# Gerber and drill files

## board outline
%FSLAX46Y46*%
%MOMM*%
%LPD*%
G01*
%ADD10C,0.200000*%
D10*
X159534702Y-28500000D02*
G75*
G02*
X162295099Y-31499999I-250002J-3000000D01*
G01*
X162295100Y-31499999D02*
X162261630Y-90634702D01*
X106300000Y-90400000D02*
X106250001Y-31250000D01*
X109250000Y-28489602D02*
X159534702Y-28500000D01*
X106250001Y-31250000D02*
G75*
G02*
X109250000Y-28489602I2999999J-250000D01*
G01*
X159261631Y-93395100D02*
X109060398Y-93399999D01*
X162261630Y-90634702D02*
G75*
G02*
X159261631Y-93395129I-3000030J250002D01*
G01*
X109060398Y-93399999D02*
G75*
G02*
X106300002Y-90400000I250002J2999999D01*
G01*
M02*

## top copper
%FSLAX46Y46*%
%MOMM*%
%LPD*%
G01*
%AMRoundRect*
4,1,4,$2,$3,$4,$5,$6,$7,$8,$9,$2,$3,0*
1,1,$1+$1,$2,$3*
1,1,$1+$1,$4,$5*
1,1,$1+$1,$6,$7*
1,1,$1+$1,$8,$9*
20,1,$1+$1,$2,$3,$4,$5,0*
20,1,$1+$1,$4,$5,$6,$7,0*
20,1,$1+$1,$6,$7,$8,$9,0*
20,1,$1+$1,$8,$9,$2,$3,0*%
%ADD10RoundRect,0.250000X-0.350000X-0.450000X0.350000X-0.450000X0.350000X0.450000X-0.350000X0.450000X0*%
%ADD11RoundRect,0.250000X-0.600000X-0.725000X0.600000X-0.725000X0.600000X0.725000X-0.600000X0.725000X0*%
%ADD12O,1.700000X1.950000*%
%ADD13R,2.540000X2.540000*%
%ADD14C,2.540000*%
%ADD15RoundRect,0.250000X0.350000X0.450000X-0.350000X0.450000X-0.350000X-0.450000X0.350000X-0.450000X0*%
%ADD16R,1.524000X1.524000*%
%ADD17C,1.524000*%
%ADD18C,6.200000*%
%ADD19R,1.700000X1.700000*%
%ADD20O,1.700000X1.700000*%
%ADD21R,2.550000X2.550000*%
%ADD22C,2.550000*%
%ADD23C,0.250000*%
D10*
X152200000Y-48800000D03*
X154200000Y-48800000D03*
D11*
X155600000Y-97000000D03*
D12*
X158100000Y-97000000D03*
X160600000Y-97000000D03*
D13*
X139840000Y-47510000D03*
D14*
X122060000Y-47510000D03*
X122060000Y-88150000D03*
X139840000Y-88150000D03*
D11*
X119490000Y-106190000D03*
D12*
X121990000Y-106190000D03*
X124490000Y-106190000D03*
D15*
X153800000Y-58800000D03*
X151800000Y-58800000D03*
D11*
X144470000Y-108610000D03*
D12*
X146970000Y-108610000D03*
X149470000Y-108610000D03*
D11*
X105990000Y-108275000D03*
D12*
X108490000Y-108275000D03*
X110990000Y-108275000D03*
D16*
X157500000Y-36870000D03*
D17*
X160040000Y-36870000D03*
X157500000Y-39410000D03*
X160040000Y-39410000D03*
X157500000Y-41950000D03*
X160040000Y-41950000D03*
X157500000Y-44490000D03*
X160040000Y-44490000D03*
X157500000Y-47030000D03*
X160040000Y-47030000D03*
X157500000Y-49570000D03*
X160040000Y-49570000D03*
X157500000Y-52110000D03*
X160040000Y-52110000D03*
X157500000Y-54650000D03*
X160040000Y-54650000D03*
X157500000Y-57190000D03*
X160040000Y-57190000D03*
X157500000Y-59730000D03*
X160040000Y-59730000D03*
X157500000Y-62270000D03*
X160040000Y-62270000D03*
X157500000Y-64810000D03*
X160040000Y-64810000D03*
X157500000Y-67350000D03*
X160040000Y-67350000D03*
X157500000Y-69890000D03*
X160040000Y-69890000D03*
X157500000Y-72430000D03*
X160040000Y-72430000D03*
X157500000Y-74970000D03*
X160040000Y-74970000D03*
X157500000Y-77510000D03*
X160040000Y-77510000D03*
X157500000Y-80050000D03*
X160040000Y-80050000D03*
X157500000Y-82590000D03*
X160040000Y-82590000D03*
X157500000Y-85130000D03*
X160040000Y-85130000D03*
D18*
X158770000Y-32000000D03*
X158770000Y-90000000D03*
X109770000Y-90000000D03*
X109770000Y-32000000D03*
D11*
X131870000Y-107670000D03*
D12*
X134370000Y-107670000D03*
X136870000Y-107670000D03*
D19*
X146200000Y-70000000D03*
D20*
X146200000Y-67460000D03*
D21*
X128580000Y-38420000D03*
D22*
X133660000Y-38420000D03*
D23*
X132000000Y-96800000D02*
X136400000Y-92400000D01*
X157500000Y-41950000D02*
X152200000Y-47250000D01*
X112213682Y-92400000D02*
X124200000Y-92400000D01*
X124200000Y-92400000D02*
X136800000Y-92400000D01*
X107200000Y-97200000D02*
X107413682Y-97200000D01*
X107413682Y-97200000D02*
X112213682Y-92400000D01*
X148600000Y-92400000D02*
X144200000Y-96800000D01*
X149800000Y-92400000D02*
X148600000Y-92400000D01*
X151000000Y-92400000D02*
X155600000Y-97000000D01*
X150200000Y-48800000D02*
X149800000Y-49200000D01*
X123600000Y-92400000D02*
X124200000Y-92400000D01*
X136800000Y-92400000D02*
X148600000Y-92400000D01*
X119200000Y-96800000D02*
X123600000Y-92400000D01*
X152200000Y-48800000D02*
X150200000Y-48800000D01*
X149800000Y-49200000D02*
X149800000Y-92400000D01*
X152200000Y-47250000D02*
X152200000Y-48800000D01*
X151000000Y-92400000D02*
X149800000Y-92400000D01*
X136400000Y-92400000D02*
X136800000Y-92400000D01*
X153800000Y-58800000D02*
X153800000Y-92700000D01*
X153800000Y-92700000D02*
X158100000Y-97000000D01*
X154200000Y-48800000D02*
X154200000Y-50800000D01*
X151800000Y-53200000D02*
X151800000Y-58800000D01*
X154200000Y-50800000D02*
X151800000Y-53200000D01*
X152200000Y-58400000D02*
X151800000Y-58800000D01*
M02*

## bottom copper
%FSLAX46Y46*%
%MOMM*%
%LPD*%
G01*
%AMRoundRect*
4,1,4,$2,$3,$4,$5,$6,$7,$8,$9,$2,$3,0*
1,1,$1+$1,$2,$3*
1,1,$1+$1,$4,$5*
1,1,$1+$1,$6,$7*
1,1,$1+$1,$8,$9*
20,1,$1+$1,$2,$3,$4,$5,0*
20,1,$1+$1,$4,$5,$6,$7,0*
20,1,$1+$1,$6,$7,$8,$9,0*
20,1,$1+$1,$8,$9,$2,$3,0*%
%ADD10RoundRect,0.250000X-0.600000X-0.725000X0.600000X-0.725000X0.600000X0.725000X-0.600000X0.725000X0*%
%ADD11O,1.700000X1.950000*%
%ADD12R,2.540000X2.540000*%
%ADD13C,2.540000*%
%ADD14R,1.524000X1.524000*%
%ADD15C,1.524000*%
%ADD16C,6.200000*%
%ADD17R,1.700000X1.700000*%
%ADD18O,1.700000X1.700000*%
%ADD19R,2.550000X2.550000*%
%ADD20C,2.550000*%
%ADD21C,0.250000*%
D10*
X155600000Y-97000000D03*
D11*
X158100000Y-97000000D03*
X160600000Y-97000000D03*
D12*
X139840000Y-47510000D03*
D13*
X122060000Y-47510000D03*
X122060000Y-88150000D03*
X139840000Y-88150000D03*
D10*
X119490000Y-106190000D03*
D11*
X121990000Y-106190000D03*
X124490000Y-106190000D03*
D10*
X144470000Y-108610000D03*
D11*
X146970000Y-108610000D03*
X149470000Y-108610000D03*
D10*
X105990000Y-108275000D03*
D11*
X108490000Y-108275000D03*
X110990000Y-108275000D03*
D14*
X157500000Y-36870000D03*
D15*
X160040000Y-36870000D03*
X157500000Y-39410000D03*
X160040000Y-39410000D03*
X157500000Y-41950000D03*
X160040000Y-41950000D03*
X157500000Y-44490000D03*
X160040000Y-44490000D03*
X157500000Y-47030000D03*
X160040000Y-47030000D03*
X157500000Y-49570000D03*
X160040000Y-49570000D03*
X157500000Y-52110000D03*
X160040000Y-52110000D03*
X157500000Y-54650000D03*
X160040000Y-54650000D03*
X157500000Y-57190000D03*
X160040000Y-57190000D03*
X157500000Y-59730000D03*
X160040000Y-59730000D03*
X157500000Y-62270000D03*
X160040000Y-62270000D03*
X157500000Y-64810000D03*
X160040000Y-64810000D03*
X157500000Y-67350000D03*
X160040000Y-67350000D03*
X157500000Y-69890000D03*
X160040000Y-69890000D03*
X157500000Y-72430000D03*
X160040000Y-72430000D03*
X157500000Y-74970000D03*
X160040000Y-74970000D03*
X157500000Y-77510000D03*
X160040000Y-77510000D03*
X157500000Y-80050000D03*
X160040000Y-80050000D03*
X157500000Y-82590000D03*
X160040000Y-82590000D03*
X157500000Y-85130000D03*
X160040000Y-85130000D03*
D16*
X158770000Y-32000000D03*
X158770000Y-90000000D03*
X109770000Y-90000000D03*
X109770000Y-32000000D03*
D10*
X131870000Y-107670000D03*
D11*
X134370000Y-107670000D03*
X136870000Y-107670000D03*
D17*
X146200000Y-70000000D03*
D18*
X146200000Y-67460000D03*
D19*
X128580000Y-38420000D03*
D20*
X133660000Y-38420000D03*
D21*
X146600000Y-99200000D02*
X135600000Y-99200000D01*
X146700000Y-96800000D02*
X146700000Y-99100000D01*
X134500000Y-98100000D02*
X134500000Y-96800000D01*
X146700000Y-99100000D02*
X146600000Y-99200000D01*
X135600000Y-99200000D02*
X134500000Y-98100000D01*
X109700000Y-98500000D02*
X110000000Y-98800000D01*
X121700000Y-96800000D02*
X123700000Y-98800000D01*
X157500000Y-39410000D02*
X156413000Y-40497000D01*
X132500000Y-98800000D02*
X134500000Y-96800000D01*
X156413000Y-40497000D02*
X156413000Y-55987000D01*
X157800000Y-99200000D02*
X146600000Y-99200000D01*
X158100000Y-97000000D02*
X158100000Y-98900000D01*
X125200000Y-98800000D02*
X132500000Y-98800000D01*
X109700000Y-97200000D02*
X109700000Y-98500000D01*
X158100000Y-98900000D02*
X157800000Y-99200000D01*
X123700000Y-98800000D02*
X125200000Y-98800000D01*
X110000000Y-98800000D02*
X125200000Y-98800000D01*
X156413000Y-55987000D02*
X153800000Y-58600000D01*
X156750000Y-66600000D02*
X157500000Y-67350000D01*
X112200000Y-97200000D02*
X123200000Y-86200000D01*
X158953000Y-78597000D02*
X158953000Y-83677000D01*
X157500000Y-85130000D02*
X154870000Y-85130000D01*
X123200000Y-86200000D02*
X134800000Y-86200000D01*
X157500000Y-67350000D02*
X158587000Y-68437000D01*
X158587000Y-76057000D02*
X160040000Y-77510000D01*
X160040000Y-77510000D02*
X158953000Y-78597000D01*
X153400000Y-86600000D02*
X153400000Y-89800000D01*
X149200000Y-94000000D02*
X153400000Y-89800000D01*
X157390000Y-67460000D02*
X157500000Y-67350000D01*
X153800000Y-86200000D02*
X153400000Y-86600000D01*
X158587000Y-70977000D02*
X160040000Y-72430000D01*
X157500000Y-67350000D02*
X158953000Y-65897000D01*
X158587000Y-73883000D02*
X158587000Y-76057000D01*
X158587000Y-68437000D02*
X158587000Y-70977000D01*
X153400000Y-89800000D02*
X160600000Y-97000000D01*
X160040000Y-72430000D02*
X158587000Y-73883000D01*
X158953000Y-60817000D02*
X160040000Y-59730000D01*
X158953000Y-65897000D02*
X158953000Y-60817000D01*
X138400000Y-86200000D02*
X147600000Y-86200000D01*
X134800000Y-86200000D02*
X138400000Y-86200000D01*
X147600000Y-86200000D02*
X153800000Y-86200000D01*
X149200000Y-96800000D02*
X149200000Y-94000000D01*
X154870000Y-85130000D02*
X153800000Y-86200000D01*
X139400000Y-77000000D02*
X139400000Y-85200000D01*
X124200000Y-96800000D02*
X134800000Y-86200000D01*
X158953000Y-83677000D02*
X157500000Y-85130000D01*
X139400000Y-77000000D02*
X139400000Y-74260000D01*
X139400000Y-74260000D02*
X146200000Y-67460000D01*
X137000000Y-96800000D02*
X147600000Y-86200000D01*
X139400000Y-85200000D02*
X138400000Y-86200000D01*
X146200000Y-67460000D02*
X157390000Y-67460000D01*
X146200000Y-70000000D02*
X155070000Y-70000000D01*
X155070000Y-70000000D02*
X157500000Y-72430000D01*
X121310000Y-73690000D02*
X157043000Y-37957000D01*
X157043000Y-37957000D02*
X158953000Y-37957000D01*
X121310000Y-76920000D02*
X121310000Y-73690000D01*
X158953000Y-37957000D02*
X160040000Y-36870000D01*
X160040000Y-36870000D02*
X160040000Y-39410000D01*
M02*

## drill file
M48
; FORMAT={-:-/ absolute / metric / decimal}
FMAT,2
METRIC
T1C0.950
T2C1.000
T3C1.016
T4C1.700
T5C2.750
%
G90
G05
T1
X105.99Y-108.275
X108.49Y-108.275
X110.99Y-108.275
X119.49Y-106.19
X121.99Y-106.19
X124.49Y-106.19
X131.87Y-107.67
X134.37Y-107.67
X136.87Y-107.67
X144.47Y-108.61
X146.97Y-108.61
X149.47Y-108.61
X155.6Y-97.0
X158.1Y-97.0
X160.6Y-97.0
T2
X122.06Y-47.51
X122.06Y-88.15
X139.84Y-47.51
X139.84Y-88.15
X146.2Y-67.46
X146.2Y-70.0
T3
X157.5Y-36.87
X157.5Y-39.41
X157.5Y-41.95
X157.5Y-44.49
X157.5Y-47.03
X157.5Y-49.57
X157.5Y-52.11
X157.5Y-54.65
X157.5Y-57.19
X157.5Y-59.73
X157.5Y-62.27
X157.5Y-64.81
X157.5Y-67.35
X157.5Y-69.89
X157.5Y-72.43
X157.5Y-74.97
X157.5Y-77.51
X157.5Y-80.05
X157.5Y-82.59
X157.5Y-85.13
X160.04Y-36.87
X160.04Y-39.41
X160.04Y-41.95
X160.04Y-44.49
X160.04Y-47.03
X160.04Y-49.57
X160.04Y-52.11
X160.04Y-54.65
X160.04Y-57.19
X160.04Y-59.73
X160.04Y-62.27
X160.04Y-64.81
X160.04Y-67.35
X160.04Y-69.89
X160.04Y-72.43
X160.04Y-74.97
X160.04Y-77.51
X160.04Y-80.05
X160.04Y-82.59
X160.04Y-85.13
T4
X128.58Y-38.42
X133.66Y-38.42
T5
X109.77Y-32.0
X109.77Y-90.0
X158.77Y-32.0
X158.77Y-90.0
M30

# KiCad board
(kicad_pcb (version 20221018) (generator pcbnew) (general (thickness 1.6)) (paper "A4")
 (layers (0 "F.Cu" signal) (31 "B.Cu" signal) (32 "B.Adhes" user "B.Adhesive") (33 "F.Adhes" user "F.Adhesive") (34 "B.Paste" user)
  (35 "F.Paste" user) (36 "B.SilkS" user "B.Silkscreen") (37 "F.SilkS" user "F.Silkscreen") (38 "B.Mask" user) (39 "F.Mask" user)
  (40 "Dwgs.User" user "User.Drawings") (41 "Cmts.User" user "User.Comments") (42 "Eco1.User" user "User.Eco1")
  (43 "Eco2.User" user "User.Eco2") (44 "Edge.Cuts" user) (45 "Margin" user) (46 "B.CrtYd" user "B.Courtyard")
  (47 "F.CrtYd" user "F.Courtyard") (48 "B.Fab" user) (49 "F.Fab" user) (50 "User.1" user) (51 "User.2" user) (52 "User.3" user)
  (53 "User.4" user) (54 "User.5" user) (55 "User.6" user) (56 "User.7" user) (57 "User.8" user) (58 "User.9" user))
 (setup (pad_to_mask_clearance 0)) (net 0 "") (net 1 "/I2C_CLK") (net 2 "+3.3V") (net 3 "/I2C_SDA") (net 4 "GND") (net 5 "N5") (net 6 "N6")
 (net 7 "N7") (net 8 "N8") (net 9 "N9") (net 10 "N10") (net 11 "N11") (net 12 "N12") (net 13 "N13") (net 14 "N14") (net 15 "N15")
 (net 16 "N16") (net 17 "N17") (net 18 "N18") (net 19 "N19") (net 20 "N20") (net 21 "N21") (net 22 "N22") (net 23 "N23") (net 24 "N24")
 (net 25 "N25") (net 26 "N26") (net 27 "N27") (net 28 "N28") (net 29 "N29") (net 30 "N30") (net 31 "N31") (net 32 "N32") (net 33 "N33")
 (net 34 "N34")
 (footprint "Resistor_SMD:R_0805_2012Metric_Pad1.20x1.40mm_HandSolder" (layer "F.Cu") (at 153.2 48.8)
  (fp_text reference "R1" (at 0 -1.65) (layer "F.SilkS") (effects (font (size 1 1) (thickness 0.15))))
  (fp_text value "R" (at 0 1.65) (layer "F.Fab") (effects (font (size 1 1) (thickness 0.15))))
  (pad "1" smd roundrect (at -1 0) (size 1.2 1.4) (layers "F.Cu" "F.Paste" "F.Mask") (roundrect_rratio 0.208333) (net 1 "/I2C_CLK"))
  (pad "2" smd roundrect (at 1 0) (size 1.2 1.4) (layers "F.Cu" "F.Paste" "F.Mask") (roundrect_rratio 0.208333) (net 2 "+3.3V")))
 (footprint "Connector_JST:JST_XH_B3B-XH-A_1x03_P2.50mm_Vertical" (layer "F.Cu") (at 155.6 97)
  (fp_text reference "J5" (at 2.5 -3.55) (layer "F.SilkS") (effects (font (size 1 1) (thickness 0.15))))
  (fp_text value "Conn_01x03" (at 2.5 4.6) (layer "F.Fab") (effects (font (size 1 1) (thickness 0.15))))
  (pad "1" thru_hole roundrect (at 0 0) (size 1.7 1.95) (drill 0.95) (layers "*.Cu" "*.Mask") (roundrect_rratio 0.147059) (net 1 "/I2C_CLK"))
  (pad "2" thru_hole oval (at 2.5 0) (size 1.7 1.95) (drill 0.95) (layers "*.Cu" "*.Mask") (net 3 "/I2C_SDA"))
  (pad "3" thru_hole oval (at 5 0) (size 1.7 1.95) (drill 0.95) (layers "*.Cu" "*.Mask") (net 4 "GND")))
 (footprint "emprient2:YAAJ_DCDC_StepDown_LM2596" (layer "F.Cu") (at 139.84 47.51 -90)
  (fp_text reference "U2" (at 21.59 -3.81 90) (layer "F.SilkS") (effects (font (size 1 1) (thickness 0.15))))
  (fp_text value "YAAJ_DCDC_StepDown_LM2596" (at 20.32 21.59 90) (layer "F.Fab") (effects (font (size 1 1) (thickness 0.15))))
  (pad "1" thru_hole rect (at 0 0 270) (size 2.54 2.54) (drill 1) (layers "*.Cu" "*.Mask") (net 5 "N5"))
  (pad "2" thru_hole circle (at 0 17.78 270) (size 2.54 2.54) (drill 1) (layers "*.Cu" "*.Mask") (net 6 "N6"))
  (pad "3" thru_hole circle (at 40.64 17.78 270) (size 2.54 2.54) (drill 1) (layers "*.Cu" "*.Mask") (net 4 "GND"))
  (pad "4" thru_hole circle (at 40.64 0 270) (size 2.54 2.54) (drill 1) (layers "*.Cu" "*.Mask") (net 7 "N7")))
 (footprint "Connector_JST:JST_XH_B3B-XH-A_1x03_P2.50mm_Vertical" (layer "F.Cu") (at 119.49 106.19)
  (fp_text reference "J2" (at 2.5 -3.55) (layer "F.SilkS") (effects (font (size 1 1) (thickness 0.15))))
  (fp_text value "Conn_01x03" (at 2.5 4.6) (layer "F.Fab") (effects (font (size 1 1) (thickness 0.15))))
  (pad "1" thru_hole roundrect (at 0 0) (size 1.7 1.95) (drill 0.95) (layers "*.Cu" "*.Mask") (roundrect_rratio 0.147059) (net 1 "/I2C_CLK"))
  (pad "2" thru_hole oval (at 2.5 0) (size 1.7 1.95) (drill 0.95) (layers "*.Cu" "*.Mask") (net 3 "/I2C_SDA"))
  (pad "3" thru_hole oval (at 5 0) (size 1.7 1.95) (drill 0.95) (layers "*.Cu" "*.Mask") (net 4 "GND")))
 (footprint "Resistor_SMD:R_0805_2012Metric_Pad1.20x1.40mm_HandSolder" (layer "F.Cu") (at 152.8 58.8 180)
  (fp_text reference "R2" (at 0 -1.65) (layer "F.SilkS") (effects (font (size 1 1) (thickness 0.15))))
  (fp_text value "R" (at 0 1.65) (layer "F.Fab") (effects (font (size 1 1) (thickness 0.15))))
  (pad "1" smd roundrect (at -1 0 180) (size 1.2 1.4) (layers "F.Cu" "F.Paste" "F.Mask") (roundrect_rratio 0.208333) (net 3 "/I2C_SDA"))
  (pad "2" smd roundrect (at 1 0 180) (size 1.2 1.4) (layers "F.Cu" "F.Paste" "F.Mask") (roundrect_rratio 0.208333) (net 2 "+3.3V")))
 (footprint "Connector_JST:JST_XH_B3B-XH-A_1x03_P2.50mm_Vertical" (layer "F.Cu") (at 144.47 108.61)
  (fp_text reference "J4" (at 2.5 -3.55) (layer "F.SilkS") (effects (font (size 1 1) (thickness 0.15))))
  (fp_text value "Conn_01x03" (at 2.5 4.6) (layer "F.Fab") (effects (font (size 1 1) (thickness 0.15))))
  (pad "1" thru_hole roundrect (at 0 0) (size 1.7 1.95) (drill 0.95) (layers "*.Cu" "*.Mask") (roundrect_rratio 0.147059) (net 1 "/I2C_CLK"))
  (pad "2" thru_hole oval (at 2.5 0) (size 1.7 1.95) (drill 0.95) (layers "*.Cu" "*.Mask") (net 3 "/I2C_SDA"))
  (pad "3" thru_hole oval (at 5 0) (size 1.7 1.95) (drill 0.95) (layers "*.Cu" "*.Mask") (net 4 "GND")))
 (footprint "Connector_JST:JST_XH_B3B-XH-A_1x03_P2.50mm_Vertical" (layer "F.Cu") (at 105.99 108.275)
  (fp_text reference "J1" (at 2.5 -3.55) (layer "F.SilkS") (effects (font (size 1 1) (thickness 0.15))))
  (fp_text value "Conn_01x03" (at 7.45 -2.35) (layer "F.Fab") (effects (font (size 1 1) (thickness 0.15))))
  (pad "1" thru_hole roundrect (at 0 0) (size 1.7 1.95) (drill 0.95) (layers "*.Cu" "*.Mask") (roundrect_rratio 0.147059) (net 1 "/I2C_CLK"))
  (pad "2" thru_hole oval (at 2.5 0) (size 1.7 1.95) (drill 0.95) (layers "*.Cu" "*.Mask") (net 3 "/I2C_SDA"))
  (pad "3" thru_hole oval (at 5 0) (size 1.7 1.95) (drill 0.95) (layers "*.Cu" "*.Mask") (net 4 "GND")))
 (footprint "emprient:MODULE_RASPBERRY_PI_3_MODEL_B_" (layer "F.Cu") (at 134.27 71 -90)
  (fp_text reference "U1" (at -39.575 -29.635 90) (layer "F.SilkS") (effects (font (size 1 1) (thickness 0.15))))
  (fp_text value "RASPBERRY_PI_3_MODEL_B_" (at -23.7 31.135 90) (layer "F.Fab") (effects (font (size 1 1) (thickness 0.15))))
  (pad "1" thru_hole rect (at -34.13 -23.23 270) (size 1.524 1.524) (drill 1.016) (layers "*.Cu" "*.Mask") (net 2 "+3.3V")
   (solder_mask_margin 0.102))
  (pad "2" thru_hole circle (at -34.13 -25.77 270) (size 1.524 1.524) (drill 1.016) (layers "*.Cu" "*.Mask") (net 7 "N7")
   (solder_mask_margin 0.102))
  (pad "3" thru_hole circle (at -31.59 -23.23 270) (size 1.524 1.524) (drill 1.016) (layers "*.Cu" "*.Mask") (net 3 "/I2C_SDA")
   (solder_mask_margin 0.102))
  (pad "4" thru_hole circle (at -31.59 -25.77 270) (size 1.524 1.524) (drill 1.016) (layers "*.Cu" "*.Mask") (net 7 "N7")
   (solder_mask_margin 0.102))
  (pad "5" thru_hole circle (at -29.05 -23.23 270) (size 1.524 1.524) (drill 1.016) (layers "*.Cu" "*.Mask") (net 1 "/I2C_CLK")
   (solder_mask_margin 0.102))
  (pad "6" thru_hole circle (at -29.05 -25.77 270) (size 1.524 1.524) (drill 1.016) (layers "*.Cu" "*.Mask") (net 4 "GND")
   (solder_mask_margin 0.102))
  (pad "7" thru_hole circle (at -26.51 -23.23 270) (size 1.524 1.524) (drill 1.016) (layers "*.Cu" "*.Mask") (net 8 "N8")
   (solder_mask_margin 0.102))
  (pad "8" thru_hole circle (at -26.51 -25.77 270) (size 1.524 1.524) (drill 1.016) (layers "*.Cu" "*.Mask") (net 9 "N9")
   (solder_mask_margin 0.102))
  (pad "9" thru_hole circle (at -23.97 -23.23 270) (size 1.524 1.524) (drill 1.016) (layers "*.Cu" "*.Mask") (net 4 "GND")
   (solder_mask_margin 0.102))
  (pad "10" thru_hole circle (at -23.97 -25.77 270) (size 1.524 1.524) (drill 1.016) (layers "*.Cu" "*.Mask") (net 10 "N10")
   (solder_mask_margin 0.102))
  (pad "11" thru_hole circle (at -21.43 -23.23 270) (size 1.524 1.524) (drill 1.016) (layers "*.Cu" "*.Mask") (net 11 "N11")
   (solder_mask_margin 0.102))
  (pad "12" thru_hole circle (at -21.43 -25.77 270) (size 1.524 1.524) (drill 1.016) (layers "*.Cu" "*.Mask") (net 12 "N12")
   (solder_mask_margin 0.102))
  (pad "13" thru_hole circle (at -18.89 -23.23 270) (size 1.524 1.524) (drill 1.016) (layers "*.Cu" "*.Mask") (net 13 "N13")
   (solder_mask_margin 0.102))
  (pad "14" thru_hole circle (at -18.89 -25.77 270) (size 1.524 1.524) (drill 1.016) (layers "*.Cu" "*.Mask") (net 4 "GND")
   (solder_mask_margin 0.102))
  (pad "15" thru_hole circle (at -16.35 -23.23 270) (size 1.524 1.524) (drill 1.016) (layers "*.Cu" "*.Mask") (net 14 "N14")
   (solder_mask_margin 0.102))
  (pad "16" thru_hole circle (at -16.35 -25.77 270) (size 1.524 1.524) (drill 1.016) (layers "*.Cu" "*.Mask") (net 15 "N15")
   (solder_mask_margin 0.102))
  (pad "17" thru_hole circle (at -13.81 -23.23 270) (size 1.524 1.524) (drill 1.016) (layers "*.Cu" "*.Mask") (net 2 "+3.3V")
   (solder_mask_margin 0.102))
  (pad "18" thru_hole circle (at -13.81 -25.77 270) (size 1.524 1.524) (drill 1.016) (layers "*.Cu" "*.Mask") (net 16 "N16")
   (solder_mask_margin 0.102))
  (pad "19" thru_hole circle (at -11.27 -23.23 270) (size 1.524 1.524) (drill 1.016) (layers "*.Cu" "*.Mask") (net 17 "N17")
   (solder_mask_margin 0.102))
  (pad "20" thru_hole circle (at -11.27 -25.77 270) (size 1.524 1.524) (drill 1.016) (layers "*.Cu" "*.Mask") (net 4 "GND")
   (solder_mask_margin 0.102))
  (pad "21" thru_hole circle (at -8.73 -23.23 270) (size 1.524 1.524) (drill 1.016) (layers "*.Cu" "*.Mask") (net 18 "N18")
   (solder_mask_margin 0.102))
  (pad "22" thru_hole circle (at -8.73 -25.77 270) (size 1.524 1.524) (drill 1.016) (layers "*.Cu" "*.Mask") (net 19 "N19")
   (solder_mask_margin 0.102))
  (pad "23" thru_hole circle (at -6.19 -23.23 270) (size 1.524 1.524) (drill 1.016) (layers "*.Cu" "*.Mask") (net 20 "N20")
   (solder_mask_margin 0.102))
  (pad "24" thru_hole circle (at -6.19 -25.77 270) (size 1.524 1.524) (drill 1.016) (layers "*.Cu" "*.Mask") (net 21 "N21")
   (solder_mask_margin 0.102))
  (pad "25" thru_hole circle (at -3.65 -23.23 270) (size 1.524 1.524) (drill 1.016) (layers "*.Cu" "*.Mask") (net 4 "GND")
   (solder_mask_margin 0.102))
  (pad "26" thru_hole circle (at -3.65 -25.77 270) (size 1.524 1.524) (drill 1.016) (layers "*.Cu" "*.Mask") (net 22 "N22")
   (solder_mask_margin 0.102))
  (pad "27" thru_hole circle (at -1.11 -23.23 270) (size 1.524 1.524) (drill 1.016) (layers "*.Cu" "*.Mask") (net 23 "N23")
   (solder_mask_margin 0.102))
  (pad "28" thru_hole circle (at -1.11 -25.77 270) (size 1.524 1.524) (drill 1.016) (layers "*.Cu" "*.Mask") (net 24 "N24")
   (solder_mask_margin 0.102))
  (pad "29" thru_hole circle (at 1.43 -23.23 270) (size 1.524 1.524) (drill 1.016) (layers "*.Cu" "*.Mask") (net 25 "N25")
   (solder_mask_margin 0.102))
  (pad "30" thru_hole circle (at 1.43 -25.77 270) (size 1.524 1.524) (drill 1.016) (layers "*.Cu" "*.Mask") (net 4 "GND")
   (solder_mask_margin 0.102))
  (pad "31" thru_hole circle (at 3.97 -23.23 270) (size 1.524 1.524) (drill 1.016) (layers "*.Cu" "*.Mask") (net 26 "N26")
   (solder_mask_margin 0.102))
  (pad "32" thru_hole circle (at 3.97 -25.77 270) (size 1.524 1.524) (drill 1.016) (layers "*.Cu" "*.Mask") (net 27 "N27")
   (solder_mask_margin 0.102))
  (pad "33" thru_hole circle (at 6.51 -23.23 270) (size 1.524 1.524) (drill 1.016) (layers "*.Cu" "*.Mask") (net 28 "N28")
   (solder_mask_margin 0.102))
  (pad "34" thru_hole circle (at 6.51 -25.77 270) (size 1.524 1.524) (drill 1.016) (layers "*.Cu" "*.Mask") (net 4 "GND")
   (solder_mask_margin 0.102))
  (pad "35" thru_hole circle (at 9.05 -23.23 270) (size 1.524 1.524) (drill 1.016) (layers "*.Cu" "*.Mask") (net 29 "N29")
   (solder_mask_margin 0.102))
  (pad "36" thru_hole circle (at 9.05 -25.77 270) (size 1.524 1.524) (drill 1.016) (layers "*.Cu" "*.Mask") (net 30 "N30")
   (solder_mask_margin 0.102))
  (pad "37" thru_hole circle (at 11.59 -23.23 270) (size 1.524 1.524) (drill 1.016) (layers "*.Cu" "*.Mask") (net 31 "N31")
   (solder_mask_margin 0.102))
  (pad "38" thru_hole circle (at 11.59 -25.77 270) (size 1.524 1.524) (drill 1.016) (layers "*.Cu" "*.Mask") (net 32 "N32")
   (solder_mask_margin 0.102))
  (pad "39" thru_hole circle (at 14.13 -23.23 270) (size 1.524 1.524) (drill 1.016) (layers "*.Cu" "*.Mask") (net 4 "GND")
   (solder_mask_margin 0.102))
  (pad "40" thru_hole circle (at 14.13 -25.77 270) (size 1.524 1.524) (drill 1.016) (layers "*.Cu" "*.Mask") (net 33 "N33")
   (solder_mask_margin 0.102))
  (pad "S1" thru_hole circle (at -39 -24.5 270) (size 6.2 6.2) (drill 2.75) (layers "*.Cu" "*.Mask") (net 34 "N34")
   (solder_mask_margin 0.102))
  (pad "S2" thru_hole circle (at 19 -24.5 270) (size 6.2 6.2) (drill 2.75) (layers "*.Cu" "*.Mask") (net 34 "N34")
   (solder_mask_margin 0.102))
  (pad "S3" thru_hole circle (at 19 24.5 270) (size 6.2 6.2) (drill 2.75) (layers "*.Cu" "*.Mask") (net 34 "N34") (solder_mask_margin 0.102))
  (pad "S4" thru_hole circle (at -39 24.5 270) (size 6.2 6.2) (drill 2.75) (layers "*.Cu" "*.Mask") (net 34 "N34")
   (solder_mask_margin 0.102)))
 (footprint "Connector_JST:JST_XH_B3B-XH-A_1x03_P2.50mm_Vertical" (layer "F.Cu") (at 131.87 107.67)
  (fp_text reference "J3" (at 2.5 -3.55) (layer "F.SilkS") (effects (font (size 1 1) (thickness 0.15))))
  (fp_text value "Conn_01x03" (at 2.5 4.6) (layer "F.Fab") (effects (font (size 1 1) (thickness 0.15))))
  (pad "1" thru_hole roundrect (at 0 0) (size 1.7 1.95) (drill 0.95) (layers "*.Cu" "*.Mask") (roundrect_rratio 0.147059) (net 1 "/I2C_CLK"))
  (pad "2" thru_hole oval (at 2.5 0) (size 1.7 1.95) (drill 0.95) (layers "*.Cu" "*.Mask") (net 3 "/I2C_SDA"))
  (pad "3" thru_hole oval (at 5 0) (size 1.7 1.95) (drill 0.95) (layers "*.Cu" "*.Mask") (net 4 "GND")))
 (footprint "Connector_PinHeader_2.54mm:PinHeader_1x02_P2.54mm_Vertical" (layer "F.Cu") (at 146.2 70 180)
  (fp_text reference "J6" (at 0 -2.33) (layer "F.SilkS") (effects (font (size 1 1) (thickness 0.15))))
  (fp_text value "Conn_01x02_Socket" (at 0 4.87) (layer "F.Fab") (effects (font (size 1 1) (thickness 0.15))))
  (pad "1" thru_hole rect (at 0 0 180) (size 1.7 1.7) (drill 1) (layers "*.Cu" "*.Mask") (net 25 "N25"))
  (pad "2" thru_hole oval (at 0 2.54 180) (size 1.7 1.7) (drill 1) (layers "*.Cu" "*.Mask") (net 4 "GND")))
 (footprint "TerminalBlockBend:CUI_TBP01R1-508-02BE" (layer "F.Cu") (at 128.58 38.42)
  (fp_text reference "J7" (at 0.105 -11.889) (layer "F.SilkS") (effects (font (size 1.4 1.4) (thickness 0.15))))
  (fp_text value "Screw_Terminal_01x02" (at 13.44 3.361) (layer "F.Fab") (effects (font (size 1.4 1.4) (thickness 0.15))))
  (pad "1" thru_hole rect (at 0 0) (size 2.55 2.55) (drill 1.7) (layers "*.Cu" "*.Mask") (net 5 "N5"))
  (pad "2" thru_hole circle (at 5.08 0) (size 2.55 2.55) (drill 1.7) (layers "*.Cu" "*.Mask") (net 6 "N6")))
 (gr_arc (start 159.534702 28.5) (mid 161.5 29.461631) (end 162.2951 31.499999) (stroke (width 0.2) (type default)) (layer "Edge.Cuts"))
 (gr_line (start 162.2951 31.499999) (end 162.26163 90.634702) (stroke (width 0.2) (type default)) (layer "Edge.Cuts"))
 (gr_line (start 106.3 90.4) (end 106.250001 31.25) (stroke (width 0.2) (type default)) (layer "Edge.Cuts"))
 (gr_line (start 109.25 28.489602) (end 159.534702 28.5) (stroke (width 0.2) (type default)) (layer "Edge.Cuts"))
 (gr_arc (start 106.250001 31.25) (mid 107.211631 29.284702) (end 109.25 28.489602) (stroke (width 0.2) (type default)) (layer "Edge.Cuts"))
 (gr_line (start 159.261631 93.3951) (end 109.060398 93.399999) (stroke (width 0.2) (type default)) (layer "Edge.Cuts"))
 (gr_arc (start 162.26163 90.634702) (mid 161.299999 92.6) (end 159.261631 93.3951) (stroke (width 0.2) (type default)) (layer "Edge.Cuts"))
 (gr_arc (start 109.060398 93.399999) (mid 107.0951 92.438368) (end 106.3 90.4) (stroke (width 0.2) (type default)) (layer "Edge.Cuts"))
 (segment (start 132 96.8) (end 136.4 92.4) (width 0.25) (layer "F.Cu") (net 1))
 (segment (start 157.5 41.95) (end 152.2 47.25) (width 0.25) (layer "F.Cu") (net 1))
 (segment (start 112.213682 92.4) (end 124.2 92.4) (width 0.25) (layer "F.Cu") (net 1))
 (segment (start 124.2 92.4) (end 136.8 92.4) (width 0.25) (layer "F.Cu") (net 1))
 (segment (start 107.2 97.2) (end 107.413682 97.2) (width 0.25) (layer "F.Cu") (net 1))
 (segment (start 107.413682 97.2) (end 112.213682 92.4) (width 0.25) (layer "F.Cu") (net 1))
 (segment (start 148.6 92.4) (end 144.2 96.8) (width 0.25) (layer "F.Cu") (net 1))
 (segment (start 149.8 92.4) (end 148.6 92.4) (width 0.25) (layer "F.Cu") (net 1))
 (segment (start 151 92.4) (end 155.6 97) (width 0.25) (layer "F.Cu") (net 1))
 (segment (start 150.2 48.8) (end 149.8 49.2) (width 0.25) (layer "F.Cu") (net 1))
 (segment (start 123.6 92.4) (end 124.2 92.4) (width 0.25) (layer "F.Cu") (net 1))
 (segment (start 136.8 92.4) (end 148.6 92.4) (width 0.25) (layer "F.Cu") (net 1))
 (segment (start 119.2 96.8) (end 123.6 92.4) (width 0.25) (layer "F.Cu") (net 1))
 (segment (start 152.2 48.8) (end 150.2 48.8) (width 0.25) (layer "F.Cu") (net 1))
 (segment (start 149.8 49.2) (end 149.8 92.4) (width 0.25) (layer "F.Cu") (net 1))
 (segment (start 152.2 47.25) (end 152.2 48.8) (width 0.25) (layer "F.Cu") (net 1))
 (segment (start 151 92.4) (end 149.8 92.4) (width 0.25) (layer "F.Cu") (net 1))
 (segment (start 136.4 92.4) (end 136.8 92.4) (width 0.25) (layer "F.Cu") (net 1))
 (segment (start 153.8 58.8) (end 153.8 92.7) (width 0.25) (layer "F.Cu") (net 3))
 (segment (start 153.8 92.7) (end 158.1 97) (width 0.25) (layer "F.Cu") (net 3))
 (segment (start 146.6 99.2) (end 135.6 99.2) (width 0.25) (layer "B.Cu") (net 3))
 (segment (start 146.7 96.8) (end 146.7 99.1) (width 0.25) (layer "B.Cu") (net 3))
 (segment (start 134.5 98.1) (end 134.5 96.8) (width 0.25) (layer "B.Cu") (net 3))
 (segment (start 146.7 99.1) (end 146.6 99.2) (width 0.25) (layer "B.Cu") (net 3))
 (segment (start 135.6 99.2) (end 134.5 98.1) (width 0.25) (layer "B.Cu") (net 3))
 (segment (start 109.7 98.5) (end 110 98.8) (width 0.25) (layer "B.Cu") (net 3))
 (segment (start 121.7 96.8) (end 123.7 98.8) (width 0.25) (layer "B.Cu") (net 3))
 (segment (start 157.5 39.41) (end 156.413 40.497) (width 0.25) (layer "B.Cu") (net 3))
 (segment (start 132.5 98.8) (end 134.5 96.8) (width 0.25) (layer "B.Cu") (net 3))
 (segment (start 156.413 40.497) (end 156.413 55.987) (width 0.25) (layer "B.Cu") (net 3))
 (segment (start 157.8 99.2) (end 146.6 99.2) (width 0.25) (layer "B.Cu") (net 3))
 (segment (start 158.1 97) (end 158.1 98.9) (width 0.25) (layer "B.Cu") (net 3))
 (segment (start 125.2 98.8) (end 132.5 98.8) (width 0.25) (layer "B.Cu") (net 3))
 (segment (start 109.7 97.2) (end 109.7 98.5) (width 0.25) (layer "B.Cu") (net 3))
 (segment (start 158.1 98.9) (end 157.8 99.2) (width 0.25) (layer "B.Cu") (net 3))
 (segment (start 123.7 98.8) (end 125.2 98.8) (width 0.25) (layer "B.Cu") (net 3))
 (segment (start 110 98.8) (end 125.2 98.8) (width 0.25) (layer "B.Cu") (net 3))
 (segment (start 156.413 55.987) (end 153.8 58.6) (width 0.25) (layer "B.Cu") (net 3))
 (segment (start 156.75 66.6) (end 157.5 67.35) (width 0.25) (layer "B.Cu") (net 4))
 (segment (start 112.2 97.2) (end 123.2 86.2) (width 0.25) (layer "B.Cu") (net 4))
 (segment (start 158.953 78.597) (end 158.953 83.677) (width 0.25) (layer "B.Cu") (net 4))
 (segment (start 157.5 85.13) (end 154.87 85.13) (width 0.25) (layer "B.Cu") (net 4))
 (segment (start 123.2 86.2) (end 134.8 86.2) (width 0.25) (layer "B.Cu") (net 4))
 (segment (start 157.5 67.35) (end 158.587 68.437) (width 0.25) (layer "B.Cu") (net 4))
 (segment (start 158.587 76.057) (end 160.04 77.51) (width 0.25) (layer "B.Cu") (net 4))
 (segment (start 160.04 77.51) (end 158.953 78.597) (width 0.25) (layer "B.Cu") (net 4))
 (segment (start 153.4 86.6) (end 153.4 89.8) (width 0.25) (layer "B.Cu") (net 4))
 (segment (start 149.2 94) (end 153.4 89.8) (width 0.25) (layer "B.Cu") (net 4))
 (segment (start 157.39 67.46) (end 157.5 67.35) (width 0.25) (layer "B.Cu") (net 4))
 (segment (start 153.8 86.2) (end 153.4 86.6) (width 0.25) (layer "B.Cu") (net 4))
 (segment (start 158.587 70.977) (end 160.04 72.43) (width 0.25) (layer "B.Cu") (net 4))
 (segment (start 157.5 67.35) (end 158.953 65.897) (width 0.25) (layer "B.Cu") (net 4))
 (segment (start 158.587 73.883) (end 158.587 76.057) (width 0.25) (layer "B.Cu") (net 4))
 (segment (start 158.587 68.437) (end 158.587 70.977) (width 0.25) (layer "B.Cu") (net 4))
 (segment (start 153.4 89.8) (end 160.6 97) (width 0.25) (layer "B.Cu") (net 4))
 (segment (start 160.04 72.43) (end 158.587 73.883) (width 0.25) (layer "B.Cu") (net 4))
 (segment (start 158.953 60.817) (end 160.04 59.73) (width 0.25) (layer "B.Cu") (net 4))
 (segment (start 158.953 65.897) (end 158.953 60.817) (width 0.25) (layer "B.Cu") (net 4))
 (segment (start 138.4 86.2) (end 147.6 86.2) (width 0.25) (layer "B.Cu") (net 4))
 (segment (start 134.8 86.2) (end 138.4 86.2) (width 0.25) (layer "B.Cu") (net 4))
 (segment (start 147.6 86.2) (end 153.8 86.2) (width 0.25) (layer "B.Cu") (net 4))
 (segment (start 149.2 96.8) (end 149.2 94) (width 0.25) (layer "B.Cu") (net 4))
 (segment (start 154.87 85.13) (end 153.8 86.2) (width 0.25) (layer "B.Cu") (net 4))
 (segment (start 139.4 77) (end 139.4 85.2) (width 0.25) (layer "B.Cu") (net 4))
 (segment (start 124.2 96.8) (end 134.8 86.2) (width 0.25) (layer "B.Cu") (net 4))
 (segment (start 158.953 83.677) (end 157.5 85.13) (width 0.25) (layer "B.Cu") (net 4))
 (segment (start 139.4 77) (end 139.4 74.26) (width 0.25) (layer "B.Cu") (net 4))
 (segment (start 139.4 74.26) (end 146.2 67.46) (width 0.25) (layer "B.Cu") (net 4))
 (segment (start 137 96.8) (end 147.6 86.2) (width 0.25) (layer "B.Cu") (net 4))
 (segment (start 139.4 85.2) (end 138.4 86.2) (width 0.25) (layer "B.Cu") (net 4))
 (segment (start 146.2 67.46) (end 157.39 67.46) (width 0.25) (layer "B.Cu") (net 4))
 (segment (start 146.2 70) (end 155.07 70) (width 0.25) (layer "B.Cu") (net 25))
 (segment (start 155.07 70) (end 157.5 72.43) (width 0.25) (layer "B.Cu") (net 25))
 (segment (start 121.31 73.69) (end 157.043 37.957) (width 0.25) (layer "B.Cu") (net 7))
 (segment (start 157.043 37.957) (end 158.953 37.957) (width 0.25) (layer "B.Cu") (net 7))
 (segment (start 121.31 76.92) (end 121.31 73.69) (width 0.25) (layer "B.Cu") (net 7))
 (segment (start 158.953 37.957) (end 160.04 36.87) (width 0.25) (layer "B.Cu") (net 7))
 (segment (start 160.04 36.87) (end 160.04 39.41) (width 0.25) (layer "B.Cu") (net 7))
 (segment (start 154.2 48.8) (end 154.2 50.8) (width 0.25) (layer "F.Cu") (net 2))
 (segment (start 151.8 53.2) (end 151.8 58.8) (width 0.25) (layer "F.Cu") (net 2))
 (segment (start 154.2 50.8) (end 151.8 53.2) (width 0.25) (layer "F.Cu") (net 2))
 (segment (start 152.2 58.4) (end 151.8 58.8) (width 0.25) (layer "F.Cu") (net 2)))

